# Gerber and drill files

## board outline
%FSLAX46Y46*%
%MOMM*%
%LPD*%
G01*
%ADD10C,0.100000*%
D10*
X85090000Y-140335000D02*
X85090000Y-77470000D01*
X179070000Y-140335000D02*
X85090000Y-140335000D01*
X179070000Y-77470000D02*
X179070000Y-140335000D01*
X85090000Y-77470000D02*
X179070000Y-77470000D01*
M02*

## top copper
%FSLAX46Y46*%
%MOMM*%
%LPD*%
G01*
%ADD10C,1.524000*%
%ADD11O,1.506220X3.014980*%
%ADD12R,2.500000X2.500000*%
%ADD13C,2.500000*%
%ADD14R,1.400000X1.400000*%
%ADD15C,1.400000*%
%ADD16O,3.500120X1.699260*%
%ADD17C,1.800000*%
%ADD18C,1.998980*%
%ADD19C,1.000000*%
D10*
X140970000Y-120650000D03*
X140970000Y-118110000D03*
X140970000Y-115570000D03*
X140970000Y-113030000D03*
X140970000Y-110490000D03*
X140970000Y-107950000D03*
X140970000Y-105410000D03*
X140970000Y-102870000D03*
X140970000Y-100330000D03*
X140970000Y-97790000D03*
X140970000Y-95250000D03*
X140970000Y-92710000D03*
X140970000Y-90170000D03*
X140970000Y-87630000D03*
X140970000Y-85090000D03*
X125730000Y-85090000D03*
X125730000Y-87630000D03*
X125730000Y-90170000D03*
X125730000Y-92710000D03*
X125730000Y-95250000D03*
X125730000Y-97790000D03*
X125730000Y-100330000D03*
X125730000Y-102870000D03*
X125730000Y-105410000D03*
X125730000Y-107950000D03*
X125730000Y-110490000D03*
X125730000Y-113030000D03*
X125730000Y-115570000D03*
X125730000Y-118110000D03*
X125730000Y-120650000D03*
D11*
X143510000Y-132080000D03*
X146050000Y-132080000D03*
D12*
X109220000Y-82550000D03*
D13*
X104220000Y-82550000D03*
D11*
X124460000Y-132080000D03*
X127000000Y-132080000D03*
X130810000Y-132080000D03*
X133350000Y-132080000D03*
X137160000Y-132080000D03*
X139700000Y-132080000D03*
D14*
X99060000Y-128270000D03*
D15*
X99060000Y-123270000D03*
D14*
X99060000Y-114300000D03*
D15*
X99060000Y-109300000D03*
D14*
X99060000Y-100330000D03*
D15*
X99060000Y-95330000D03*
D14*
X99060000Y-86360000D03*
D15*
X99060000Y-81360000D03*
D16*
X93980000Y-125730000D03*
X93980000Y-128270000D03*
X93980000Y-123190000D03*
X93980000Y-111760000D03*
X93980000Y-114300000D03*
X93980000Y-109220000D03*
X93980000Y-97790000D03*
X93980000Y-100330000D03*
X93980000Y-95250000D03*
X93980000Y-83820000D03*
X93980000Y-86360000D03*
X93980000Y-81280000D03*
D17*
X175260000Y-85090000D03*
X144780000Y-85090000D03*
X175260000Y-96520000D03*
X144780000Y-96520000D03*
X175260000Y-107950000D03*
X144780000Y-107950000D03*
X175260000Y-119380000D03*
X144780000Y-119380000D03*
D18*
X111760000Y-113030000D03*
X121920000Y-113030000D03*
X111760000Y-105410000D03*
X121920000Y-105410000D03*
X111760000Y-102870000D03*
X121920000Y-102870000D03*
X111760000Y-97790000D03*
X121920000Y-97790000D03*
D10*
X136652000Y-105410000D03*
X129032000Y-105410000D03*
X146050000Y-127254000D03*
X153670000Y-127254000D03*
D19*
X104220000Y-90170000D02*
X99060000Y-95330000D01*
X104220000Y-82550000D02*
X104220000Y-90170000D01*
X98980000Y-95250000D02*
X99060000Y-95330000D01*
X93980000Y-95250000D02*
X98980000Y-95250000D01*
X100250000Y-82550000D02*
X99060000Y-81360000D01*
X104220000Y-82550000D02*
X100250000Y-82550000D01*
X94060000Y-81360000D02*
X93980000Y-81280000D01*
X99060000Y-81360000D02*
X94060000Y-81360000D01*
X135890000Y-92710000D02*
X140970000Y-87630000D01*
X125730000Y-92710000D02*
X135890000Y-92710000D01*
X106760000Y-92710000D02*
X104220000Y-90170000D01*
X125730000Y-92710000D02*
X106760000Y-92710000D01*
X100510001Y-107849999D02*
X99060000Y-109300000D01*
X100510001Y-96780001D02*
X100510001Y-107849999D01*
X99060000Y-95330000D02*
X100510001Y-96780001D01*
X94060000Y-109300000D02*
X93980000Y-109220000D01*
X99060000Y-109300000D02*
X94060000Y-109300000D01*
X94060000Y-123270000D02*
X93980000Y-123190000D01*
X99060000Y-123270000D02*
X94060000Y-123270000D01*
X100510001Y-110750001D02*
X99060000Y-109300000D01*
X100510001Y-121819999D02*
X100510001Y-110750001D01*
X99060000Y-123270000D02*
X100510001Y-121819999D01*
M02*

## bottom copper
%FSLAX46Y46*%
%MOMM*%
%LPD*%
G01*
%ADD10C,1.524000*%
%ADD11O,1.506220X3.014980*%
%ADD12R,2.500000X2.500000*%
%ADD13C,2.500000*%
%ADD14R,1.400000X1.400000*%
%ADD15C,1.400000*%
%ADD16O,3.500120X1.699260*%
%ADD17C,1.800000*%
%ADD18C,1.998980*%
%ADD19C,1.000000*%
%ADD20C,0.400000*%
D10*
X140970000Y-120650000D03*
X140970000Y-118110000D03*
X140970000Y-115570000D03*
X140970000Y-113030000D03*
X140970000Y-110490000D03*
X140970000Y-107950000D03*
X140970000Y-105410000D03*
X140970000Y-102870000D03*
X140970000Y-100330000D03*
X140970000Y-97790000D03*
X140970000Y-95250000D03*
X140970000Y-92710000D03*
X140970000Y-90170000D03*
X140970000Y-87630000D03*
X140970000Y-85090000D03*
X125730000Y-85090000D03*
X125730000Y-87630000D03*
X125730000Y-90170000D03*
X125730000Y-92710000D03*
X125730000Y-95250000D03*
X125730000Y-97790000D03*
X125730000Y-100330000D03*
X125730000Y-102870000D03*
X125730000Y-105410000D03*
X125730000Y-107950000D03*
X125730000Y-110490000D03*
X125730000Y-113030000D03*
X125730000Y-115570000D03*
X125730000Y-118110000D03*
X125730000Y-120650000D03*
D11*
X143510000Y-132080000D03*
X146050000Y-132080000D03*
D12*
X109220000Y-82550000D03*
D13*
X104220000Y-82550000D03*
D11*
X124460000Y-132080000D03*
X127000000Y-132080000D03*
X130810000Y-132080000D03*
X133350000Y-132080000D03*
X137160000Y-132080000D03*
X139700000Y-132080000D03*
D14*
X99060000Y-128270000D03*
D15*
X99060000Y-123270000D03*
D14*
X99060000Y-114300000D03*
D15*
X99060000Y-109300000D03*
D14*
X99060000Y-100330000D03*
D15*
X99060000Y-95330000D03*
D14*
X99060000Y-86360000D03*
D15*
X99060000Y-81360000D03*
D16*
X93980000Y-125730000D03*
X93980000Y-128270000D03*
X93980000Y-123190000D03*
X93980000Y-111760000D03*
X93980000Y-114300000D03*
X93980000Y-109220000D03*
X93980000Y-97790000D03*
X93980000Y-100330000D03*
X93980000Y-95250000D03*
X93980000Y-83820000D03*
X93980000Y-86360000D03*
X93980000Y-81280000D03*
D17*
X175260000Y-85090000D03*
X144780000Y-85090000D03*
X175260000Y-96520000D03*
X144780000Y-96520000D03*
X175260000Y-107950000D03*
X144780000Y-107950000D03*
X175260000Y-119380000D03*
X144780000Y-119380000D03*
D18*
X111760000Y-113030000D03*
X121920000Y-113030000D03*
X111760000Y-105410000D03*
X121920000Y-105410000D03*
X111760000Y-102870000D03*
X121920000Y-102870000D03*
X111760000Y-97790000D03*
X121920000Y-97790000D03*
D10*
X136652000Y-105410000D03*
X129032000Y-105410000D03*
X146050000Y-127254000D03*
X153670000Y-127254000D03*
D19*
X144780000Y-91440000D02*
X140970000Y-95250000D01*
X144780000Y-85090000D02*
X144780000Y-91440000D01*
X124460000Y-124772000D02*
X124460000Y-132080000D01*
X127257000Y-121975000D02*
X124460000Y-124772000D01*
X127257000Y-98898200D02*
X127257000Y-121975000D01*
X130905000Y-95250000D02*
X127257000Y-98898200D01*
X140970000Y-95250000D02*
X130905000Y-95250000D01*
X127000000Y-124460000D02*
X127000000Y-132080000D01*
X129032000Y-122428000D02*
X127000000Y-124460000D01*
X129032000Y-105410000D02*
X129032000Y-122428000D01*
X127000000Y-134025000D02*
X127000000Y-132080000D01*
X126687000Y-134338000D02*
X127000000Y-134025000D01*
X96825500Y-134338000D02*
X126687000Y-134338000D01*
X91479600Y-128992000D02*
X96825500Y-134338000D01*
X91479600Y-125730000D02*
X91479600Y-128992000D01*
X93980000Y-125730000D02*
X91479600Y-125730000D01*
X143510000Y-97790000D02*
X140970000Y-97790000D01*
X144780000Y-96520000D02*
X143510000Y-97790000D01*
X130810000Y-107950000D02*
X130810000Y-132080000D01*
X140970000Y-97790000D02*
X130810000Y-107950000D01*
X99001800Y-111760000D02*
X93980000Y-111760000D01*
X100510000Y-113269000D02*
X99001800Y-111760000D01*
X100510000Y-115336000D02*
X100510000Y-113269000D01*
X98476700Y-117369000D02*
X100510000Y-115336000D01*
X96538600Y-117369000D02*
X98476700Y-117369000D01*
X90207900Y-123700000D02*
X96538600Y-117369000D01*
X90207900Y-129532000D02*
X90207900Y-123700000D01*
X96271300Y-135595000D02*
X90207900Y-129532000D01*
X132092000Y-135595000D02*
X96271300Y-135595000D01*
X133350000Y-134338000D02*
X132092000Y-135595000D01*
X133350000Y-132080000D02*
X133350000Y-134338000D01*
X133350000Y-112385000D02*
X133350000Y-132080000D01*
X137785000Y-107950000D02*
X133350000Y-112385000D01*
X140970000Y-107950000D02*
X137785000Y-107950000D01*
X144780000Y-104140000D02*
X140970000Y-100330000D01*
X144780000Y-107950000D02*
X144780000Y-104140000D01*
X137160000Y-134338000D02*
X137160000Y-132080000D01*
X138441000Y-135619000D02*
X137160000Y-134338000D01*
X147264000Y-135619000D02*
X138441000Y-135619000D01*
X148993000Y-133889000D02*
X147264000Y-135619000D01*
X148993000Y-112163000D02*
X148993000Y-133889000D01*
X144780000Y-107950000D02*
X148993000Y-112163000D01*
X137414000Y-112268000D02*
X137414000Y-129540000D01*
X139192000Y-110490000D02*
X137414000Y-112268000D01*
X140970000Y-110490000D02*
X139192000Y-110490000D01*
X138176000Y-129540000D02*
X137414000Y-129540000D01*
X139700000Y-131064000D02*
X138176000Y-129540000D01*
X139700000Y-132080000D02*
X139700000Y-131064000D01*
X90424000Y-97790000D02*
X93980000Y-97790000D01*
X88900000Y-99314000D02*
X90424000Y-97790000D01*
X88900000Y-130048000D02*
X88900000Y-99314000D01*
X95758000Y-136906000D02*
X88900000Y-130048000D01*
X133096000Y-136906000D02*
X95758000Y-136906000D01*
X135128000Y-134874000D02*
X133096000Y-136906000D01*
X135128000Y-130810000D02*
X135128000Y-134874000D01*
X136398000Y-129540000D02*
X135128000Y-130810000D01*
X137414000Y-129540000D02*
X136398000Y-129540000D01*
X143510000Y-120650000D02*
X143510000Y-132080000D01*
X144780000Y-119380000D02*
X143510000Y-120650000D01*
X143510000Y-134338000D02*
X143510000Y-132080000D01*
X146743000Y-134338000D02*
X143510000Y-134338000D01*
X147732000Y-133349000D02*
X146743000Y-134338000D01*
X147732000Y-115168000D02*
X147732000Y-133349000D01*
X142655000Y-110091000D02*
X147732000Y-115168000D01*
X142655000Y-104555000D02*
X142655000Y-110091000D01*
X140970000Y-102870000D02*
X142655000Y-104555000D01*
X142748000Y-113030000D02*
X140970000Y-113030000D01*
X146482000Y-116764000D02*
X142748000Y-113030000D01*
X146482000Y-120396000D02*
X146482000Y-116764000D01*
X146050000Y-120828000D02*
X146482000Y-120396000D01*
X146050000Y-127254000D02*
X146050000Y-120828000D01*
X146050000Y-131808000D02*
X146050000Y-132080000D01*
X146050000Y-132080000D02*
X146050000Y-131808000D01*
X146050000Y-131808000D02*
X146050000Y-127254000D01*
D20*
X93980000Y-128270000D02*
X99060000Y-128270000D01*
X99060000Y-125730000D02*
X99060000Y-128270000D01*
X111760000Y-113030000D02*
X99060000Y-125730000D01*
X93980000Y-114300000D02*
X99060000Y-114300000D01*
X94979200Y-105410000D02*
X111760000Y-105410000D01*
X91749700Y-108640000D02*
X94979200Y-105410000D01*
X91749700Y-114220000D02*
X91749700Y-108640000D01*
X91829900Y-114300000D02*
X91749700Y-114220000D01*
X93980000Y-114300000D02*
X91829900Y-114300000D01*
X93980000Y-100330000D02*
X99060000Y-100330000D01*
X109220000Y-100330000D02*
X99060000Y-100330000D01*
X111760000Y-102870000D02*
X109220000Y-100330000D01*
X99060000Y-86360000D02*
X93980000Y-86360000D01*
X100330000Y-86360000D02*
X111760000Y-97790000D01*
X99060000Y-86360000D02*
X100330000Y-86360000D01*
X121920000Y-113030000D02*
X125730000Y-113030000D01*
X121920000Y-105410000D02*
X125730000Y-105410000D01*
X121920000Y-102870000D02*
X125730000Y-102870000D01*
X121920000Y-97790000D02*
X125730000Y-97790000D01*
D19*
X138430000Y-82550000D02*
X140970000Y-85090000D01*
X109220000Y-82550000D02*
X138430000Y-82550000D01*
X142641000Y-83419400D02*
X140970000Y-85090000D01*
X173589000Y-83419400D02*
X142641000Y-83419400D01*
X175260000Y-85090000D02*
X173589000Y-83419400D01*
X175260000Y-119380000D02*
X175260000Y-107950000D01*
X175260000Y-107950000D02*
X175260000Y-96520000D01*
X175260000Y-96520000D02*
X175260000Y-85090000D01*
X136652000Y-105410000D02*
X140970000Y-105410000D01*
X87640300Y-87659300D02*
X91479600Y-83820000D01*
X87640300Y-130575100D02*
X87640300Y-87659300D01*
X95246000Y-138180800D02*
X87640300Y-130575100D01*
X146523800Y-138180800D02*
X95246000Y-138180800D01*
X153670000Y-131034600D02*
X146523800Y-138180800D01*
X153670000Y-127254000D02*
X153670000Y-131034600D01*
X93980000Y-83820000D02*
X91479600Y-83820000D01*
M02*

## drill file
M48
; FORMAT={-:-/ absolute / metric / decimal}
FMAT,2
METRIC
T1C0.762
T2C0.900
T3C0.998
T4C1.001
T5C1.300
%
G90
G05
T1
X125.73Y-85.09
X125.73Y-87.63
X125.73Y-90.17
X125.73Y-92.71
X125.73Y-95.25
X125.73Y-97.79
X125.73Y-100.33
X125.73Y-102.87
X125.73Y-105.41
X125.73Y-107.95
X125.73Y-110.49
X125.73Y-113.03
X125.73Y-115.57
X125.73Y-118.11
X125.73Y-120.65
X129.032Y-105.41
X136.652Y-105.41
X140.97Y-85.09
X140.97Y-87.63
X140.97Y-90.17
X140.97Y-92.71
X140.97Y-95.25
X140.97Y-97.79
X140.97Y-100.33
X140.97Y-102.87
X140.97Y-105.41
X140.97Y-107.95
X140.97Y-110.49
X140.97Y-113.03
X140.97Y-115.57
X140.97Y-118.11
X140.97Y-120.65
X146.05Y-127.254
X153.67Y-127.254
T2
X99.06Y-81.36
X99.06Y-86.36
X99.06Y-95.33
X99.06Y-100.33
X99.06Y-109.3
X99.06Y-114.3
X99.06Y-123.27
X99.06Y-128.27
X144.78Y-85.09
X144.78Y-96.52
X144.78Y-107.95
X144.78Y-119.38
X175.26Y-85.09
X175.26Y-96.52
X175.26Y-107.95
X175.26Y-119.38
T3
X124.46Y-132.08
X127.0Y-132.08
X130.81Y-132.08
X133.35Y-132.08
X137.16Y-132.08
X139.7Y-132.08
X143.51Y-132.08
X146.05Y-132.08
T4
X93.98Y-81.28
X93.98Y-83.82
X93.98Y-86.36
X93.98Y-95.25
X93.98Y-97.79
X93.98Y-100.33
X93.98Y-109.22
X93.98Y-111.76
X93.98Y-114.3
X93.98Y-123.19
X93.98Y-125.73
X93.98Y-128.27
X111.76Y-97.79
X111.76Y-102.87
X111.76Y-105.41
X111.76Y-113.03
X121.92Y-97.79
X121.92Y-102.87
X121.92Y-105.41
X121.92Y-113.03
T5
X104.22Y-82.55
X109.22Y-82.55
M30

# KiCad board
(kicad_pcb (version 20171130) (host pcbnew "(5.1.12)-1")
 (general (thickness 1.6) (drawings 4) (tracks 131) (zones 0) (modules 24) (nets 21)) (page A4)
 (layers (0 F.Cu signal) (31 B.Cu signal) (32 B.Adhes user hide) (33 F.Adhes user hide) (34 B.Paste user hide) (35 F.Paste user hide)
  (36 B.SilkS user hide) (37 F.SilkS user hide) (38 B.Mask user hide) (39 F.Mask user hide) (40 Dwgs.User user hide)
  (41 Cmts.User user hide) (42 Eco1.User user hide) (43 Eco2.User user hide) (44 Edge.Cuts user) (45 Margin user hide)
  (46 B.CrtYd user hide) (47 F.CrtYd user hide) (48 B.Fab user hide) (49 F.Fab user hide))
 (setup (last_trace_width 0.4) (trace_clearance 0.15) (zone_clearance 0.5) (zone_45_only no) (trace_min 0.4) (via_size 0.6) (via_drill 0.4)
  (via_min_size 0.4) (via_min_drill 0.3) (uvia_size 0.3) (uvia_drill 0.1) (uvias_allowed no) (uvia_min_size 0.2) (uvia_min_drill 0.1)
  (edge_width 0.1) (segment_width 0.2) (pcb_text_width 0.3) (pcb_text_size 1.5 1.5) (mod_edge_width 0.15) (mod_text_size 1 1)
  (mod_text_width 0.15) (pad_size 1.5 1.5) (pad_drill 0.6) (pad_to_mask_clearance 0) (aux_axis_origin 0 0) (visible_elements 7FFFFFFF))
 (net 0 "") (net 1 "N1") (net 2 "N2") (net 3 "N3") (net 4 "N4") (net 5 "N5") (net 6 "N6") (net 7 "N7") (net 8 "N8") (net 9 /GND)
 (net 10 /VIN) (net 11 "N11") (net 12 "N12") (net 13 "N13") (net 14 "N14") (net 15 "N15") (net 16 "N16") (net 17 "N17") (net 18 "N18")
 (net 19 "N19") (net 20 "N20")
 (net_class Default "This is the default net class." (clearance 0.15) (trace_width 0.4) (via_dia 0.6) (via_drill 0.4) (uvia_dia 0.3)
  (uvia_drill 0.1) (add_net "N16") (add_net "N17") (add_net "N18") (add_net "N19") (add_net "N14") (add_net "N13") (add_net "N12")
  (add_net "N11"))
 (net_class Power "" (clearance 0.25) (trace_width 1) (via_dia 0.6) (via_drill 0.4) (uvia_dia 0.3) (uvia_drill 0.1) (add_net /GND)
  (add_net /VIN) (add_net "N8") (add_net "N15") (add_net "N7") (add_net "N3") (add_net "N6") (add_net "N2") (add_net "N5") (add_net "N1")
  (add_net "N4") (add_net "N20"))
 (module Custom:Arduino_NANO (layer F.Cu) (at 140.97 120.65 90)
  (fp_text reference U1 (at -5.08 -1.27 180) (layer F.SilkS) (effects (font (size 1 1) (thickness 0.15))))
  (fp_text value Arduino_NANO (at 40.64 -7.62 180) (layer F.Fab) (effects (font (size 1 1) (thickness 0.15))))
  (pad 1 thru_hole circle (at 0 0 90) (size 1.524 1.524) (drill 0.762) (layers *.Cu *.Mask))
  (pad 2 thru_hole circle (at 2.54 0 90) (size 1.524 1.524) (drill 0.762) (layers *.Cu *.Mask))
  (pad 3 thru_hole circle (at 5.08 0 90) (size 1.524 1.524) (drill 0.762) (layers *.Cu *.Mask))
  (pad 4 thru_hole circle (at 7.62 0 90) (size 1.524 1.524) (drill 0.762) (layers *.Cu *.Mask) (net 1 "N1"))
  (pad 5 thru_hole circle (at 10.16 0 90) (size 1.524 1.524) (drill 0.762) (layers *.Cu *.Mask) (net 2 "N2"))
  (pad 6 thru_hole circle (at 12.7 0 90) (size 1.524 1.524) (drill 0.762) (layers *.Cu *.Mask) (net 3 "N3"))
  (pad 7 thru_hole circle (at 15.24 0 90) (size 1.524 1.524) (drill 0.762) (layers *.Cu *.Mask) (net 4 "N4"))
  (pad 8 thru_hole circle (at 17.78 0 90) (size 1.524 1.524) (drill 0.762) (layers *.Cu *.Mask) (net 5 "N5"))
  (pad 9 thru_hole circle (at 20.32 0 90) (size 1.524 1.524) (drill 0.762) (layers *.Cu *.Mask) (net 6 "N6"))
  (pad 10 thru_hole circle (at 22.86 0 90) (size 1.524 1.524) (drill 0.762) (layers *.Cu *.Mask) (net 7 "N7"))
  (pad 11 thru_hole circle (at 25.4 0 90) (size 1.524 1.524) (drill 0.762) (layers *.Cu *.Mask) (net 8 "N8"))
  (pad 12 thru_hole circle (at 27.94 0 90) (size 1.524 1.524) (drill 0.762) (layers *.Cu *.Mask))
  (pad 13 thru_hole circle (at 30.48 0 90) (size 1.524 1.524) (drill 0.762) (layers *.Cu *.Mask))
  (pad 14 thru_hole circle (at 33.02 0 90) (size 1.524 1.524) (drill 0.762) (layers *.Cu *.Mask) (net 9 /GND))
  (pad 15 thru_hole circle (at 35.56 0 90) (size 1.524 1.524) (drill 0.762) (layers *.Cu *.Mask) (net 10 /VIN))
  (pad 16 thru_hole circle (at 35.56 -15.24 90) (size 1.524 1.524) (drill 0.762) (layers *.Cu *.Mask))
  (pad 17 thru_hole circle (at 33.02 -15.24 90) (size 1.524 1.524) (drill 0.762) (layers *.Cu *.Mask))
  (pad 18 thru_hole circle (at 30.48 -15.24 90) (size 1.524 1.524) (drill 0.762) (layers *.Cu *.Mask))
  (pad 19 thru_hole circle (at 27.94 -15.24 90) (size 1.524 1.524) (drill 0.762) (layers *.Cu *.Mask) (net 9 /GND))
  (pad 20 thru_hole circle (at 25.4 -15.24 90) (size 1.524 1.524) (drill 0.762) (layers *.Cu *.Mask))
  (pad 21 thru_hole circle (at 22.86 -15.24 90) (size 1.524 1.524) (drill 0.762) (layers *.Cu *.Mask) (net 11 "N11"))
  (pad 22 thru_hole circle (at 20.32 -15.24 90) (size 1.524 1.524) (drill 0.762) (layers *.Cu *.Mask))
  (pad 23 thru_hole circle (at 17.78 -15.24 90) (size 1.524 1.524) (drill 0.762) (layers *.Cu *.Mask) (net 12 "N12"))
  (pad 24 thru_hole circle (at 15.24 -15.24 90) (size 1.524 1.524) (drill 0.762) (layers *.Cu *.Mask) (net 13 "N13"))
  (pad 25 thru_hole circle (at 12.7 -15.24 90) (size 1.524 1.524) (drill 0.762) (layers *.Cu *.Mask))
  (pad 26 thru_hole circle (at 10.16 -15.24 90) (size 1.524 1.524) (drill 0.762) (layers *.Cu *.Mask))
  (pad 27 thru_hole circle (at 7.62 -15.24 90) (size 1.524 1.524) (drill 0.762) (layers *.Cu *.Mask) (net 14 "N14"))
  (pad 28 thru_hole circle (at 5.08 -15.24 90) (size 1.524 1.524) (drill 0.762) (layers *.Cu *.Mask))
  (pad 29 thru_hole circle (at 2.54 -15.24 90) (size 1.524 1.524) (drill 0.762) (layers *.Cu *.Mask))
  (pad 30 thru_hole circle (at 0 -15.24 90) (size 1.524 1.524) (drill 0.762) (layers *.Cu *.Mask)))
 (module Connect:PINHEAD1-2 (layer F.Cu) (at 144.78 132.08)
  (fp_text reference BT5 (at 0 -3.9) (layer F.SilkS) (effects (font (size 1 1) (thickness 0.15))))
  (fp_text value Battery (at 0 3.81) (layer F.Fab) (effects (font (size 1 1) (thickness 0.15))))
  (pad 1 thru_hole oval (at -1.27 0) (size 1.50622 3.01498) (drill 0.99822) (layers *.Cu *.Mask) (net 5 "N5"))
  (pad 2 thru_hole oval (at 1.27 0) (size 1.50622 3.01498) (drill 0.99822) (layers *.Cu *.Mask) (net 1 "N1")))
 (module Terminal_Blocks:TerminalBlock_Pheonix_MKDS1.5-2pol (layer F.Cu) (at 109.22 82.55 180)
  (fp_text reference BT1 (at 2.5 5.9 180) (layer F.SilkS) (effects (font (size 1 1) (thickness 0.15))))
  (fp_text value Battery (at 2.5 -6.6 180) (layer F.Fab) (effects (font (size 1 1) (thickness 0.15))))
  (pad 1 thru_hole rect (at 0 0 180) (size 2.5 2.5) (drill 1.3) (layers *.Cu *.Mask F.SilkS) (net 10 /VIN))
  (pad 2 thru_hole circle (at 5 0 180) (size 2.5 2.5) (drill 1.3) (layers *.Cu *.Mask F.SilkS) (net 9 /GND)))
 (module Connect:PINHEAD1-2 (layer F.Cu) (at 125.73 132.08)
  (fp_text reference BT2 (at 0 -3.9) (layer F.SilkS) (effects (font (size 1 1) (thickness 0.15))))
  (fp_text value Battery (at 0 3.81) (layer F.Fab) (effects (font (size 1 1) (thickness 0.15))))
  (pad 1 thru_hole oval (at -1.27 0) (size 1.50622 3.01498) (drill 0.99822) (layers *.Cu *.Mask) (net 8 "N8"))
  (pad 2 thru_hole oval (at 1.27 0) (size 1.50622 3.01498) (drill 0.99822) (layers *.Cu *.Mask) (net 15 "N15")))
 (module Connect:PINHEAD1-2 (layer F.Cu) (at 132.08 132.08)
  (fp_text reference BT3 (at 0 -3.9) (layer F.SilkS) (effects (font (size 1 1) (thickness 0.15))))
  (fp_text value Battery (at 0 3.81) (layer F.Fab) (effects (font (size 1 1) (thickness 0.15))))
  (pad 1 thru_hole oval (at -1.27 0) (size 1.50622 3.01498) (drill 0.99822) (layers *.Cu *.Mask) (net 7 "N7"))
  (pad 2 thru_hole oval (at 1.27 0) (size 1.50622 3.01498) (drill 0.99822) (layers *.Cu *.Mask) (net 3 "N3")))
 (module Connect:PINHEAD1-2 (layer F.Cu) (at 138.43 132.08)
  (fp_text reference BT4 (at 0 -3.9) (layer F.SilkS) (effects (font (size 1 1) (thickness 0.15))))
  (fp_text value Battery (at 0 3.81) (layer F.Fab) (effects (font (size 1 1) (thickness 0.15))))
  (pad 1 thru_hole oval (at -1.27 0) (size 1.50622 3.01498) (drill 0.99822) (layers *.Cu *.Mask) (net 6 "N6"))
  (pad 2 thru_hole oval (at 1.27 0) (size 1.50622 3.01498) (drill 0.99822) (layers *.Cu *.Mask) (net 2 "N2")))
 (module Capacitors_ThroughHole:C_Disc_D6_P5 (layer F.Cu) (at 99.06 128.27 90)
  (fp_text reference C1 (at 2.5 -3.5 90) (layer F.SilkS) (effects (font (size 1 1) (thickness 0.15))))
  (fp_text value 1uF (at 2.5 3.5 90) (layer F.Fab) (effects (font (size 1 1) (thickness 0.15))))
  (pad 1 thru_hole rect (at 0 0 90) (size 1.4 1.4) (drill 0.9) (layers *.Cu *.Mask F.SilkS) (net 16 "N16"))
  (pad 2 thru_hole circle (at 5 0 90) (size 1.4 1.4) (drill 0.9) (layers *.Cu *.Mask F.SilkS) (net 9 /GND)))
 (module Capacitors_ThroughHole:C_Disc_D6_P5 (layer F.Cu) (at 99.06 114.3 90)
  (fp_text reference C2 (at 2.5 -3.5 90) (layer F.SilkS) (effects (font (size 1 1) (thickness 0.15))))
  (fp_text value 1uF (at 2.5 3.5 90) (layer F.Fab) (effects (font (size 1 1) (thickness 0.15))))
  (pad 1 thru_hole rect (at 0 0 90) (size 1.4 1.4) (drill 0.9) (layers *.Cu *.Mask F.SilkS) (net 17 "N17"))
  (pad 2 thru_hole circle (at 5 0 90) (size 1.4 1.4) (drill 0.9) (layers *.Cu *.Mask F.SilkS) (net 9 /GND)))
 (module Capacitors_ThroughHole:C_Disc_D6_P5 (layer F.Cu) (at 99.06 100.33 90)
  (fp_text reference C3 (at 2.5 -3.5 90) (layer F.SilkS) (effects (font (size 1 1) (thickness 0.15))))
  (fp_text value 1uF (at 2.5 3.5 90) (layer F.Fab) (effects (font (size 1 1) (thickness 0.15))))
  (pad 1 thru_hole rect (at 0 0 90) (size 1.4 1.4) (drill 0.9) (layers *.Cu *.Mask F.SilkS) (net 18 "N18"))
  (pad 2 thru_hole circle (at 5 0 90) (size 1.4 1.4) (drill 0.9) (layers *.Cu *.Mask F.SilkS) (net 9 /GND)))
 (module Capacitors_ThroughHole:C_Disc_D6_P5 (layer F.Cu) (at 99.06 86.36 90)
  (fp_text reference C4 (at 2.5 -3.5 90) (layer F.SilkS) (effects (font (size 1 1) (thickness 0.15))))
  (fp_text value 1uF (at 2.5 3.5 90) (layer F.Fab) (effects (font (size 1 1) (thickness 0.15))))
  (pad 1 thru_hole rect (at 0 0 90) (size 1.4 1.4) (drill 0.9) (layers *.Cu *.Mask F.SilkS) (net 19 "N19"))
  (pad 2 thru_hole circle (at 5 0 90) (size 1.4 1.4) (drill 0.9) (layers *.Cu *.Mask F.SilkS) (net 9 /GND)))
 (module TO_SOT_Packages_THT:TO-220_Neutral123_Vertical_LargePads (layer F.Cu) (at 93.98 125.73 90)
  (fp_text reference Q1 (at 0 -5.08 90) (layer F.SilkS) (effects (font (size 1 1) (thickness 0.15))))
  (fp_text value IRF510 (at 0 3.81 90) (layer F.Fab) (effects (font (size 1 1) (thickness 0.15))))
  (pad 2 thru_hole oval (at 0 0 180) (size 3.50012 1.69926) (drill 1.00076) (layers *.Cu *.Mask F.SilkS) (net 15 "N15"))
  (pad 1 thru_hole oval (at -2.54 0 180) (size 3.50012 1.69926) (drill 1.00076) (layers *.Cu *.Mask F.SilkS) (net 16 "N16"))
  (pad 3 thru_hole oval (at 2.54 0 180) (size 3.50012 1.69926) (drill 1.00076) (layers *.Cu *.Mask F.SilkS) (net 9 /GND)))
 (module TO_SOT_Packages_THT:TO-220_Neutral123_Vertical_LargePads (layer F.Cu) (at 93.98 111.76 90)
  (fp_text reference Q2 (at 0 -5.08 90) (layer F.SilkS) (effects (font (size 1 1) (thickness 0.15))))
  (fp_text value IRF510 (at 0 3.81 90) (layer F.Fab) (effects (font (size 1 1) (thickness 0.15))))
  (pad 2 thru_hole oval (at 0 0 180) (size 3.50012 1.69926) (drill 1.00076) (layers *.Cu *.Mask F.SilkS) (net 3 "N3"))
  (pad 1 thru_hole oval (at -2.54 0 180) (size 3.50012 1.69926) (drill 1.00076) (layers *.Cu *.Mask F.SilkS) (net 17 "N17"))
  (pad 3 thru_hole oval (at 2.54 0 180) (size 3.50012 1.69926) (drill 1.00076) (layers *.Cu *.Mask F.SilkS) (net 9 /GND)))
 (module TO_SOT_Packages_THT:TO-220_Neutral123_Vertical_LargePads (layer F.Cu) (at 93.98 97.79 90)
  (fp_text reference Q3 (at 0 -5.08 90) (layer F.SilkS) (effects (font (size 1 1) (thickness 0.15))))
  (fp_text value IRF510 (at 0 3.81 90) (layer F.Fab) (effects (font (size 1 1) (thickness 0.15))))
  (pad 2 thru_hole oval (at 0 0 180) (size 3.50012 1.69926) (drill 1.00076) (layers *.Cu *.Mask F.SilkS) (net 2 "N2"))
  (pad 1 thru_hole oval (at -2.54 0 180) (size 3.50012 1.69926) (drill 1.00076) (layers *.Cu *.Mask F.SilkS) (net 18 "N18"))
  (pad 3 thru_hole oval (at 2.54 0 180) (size 3.50012 1.69926) (drill 1.00076) (layers *.Cu *.Mask F.SilkS) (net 9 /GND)))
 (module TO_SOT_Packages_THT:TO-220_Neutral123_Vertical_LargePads (layer F.Cu) (at 93.98 83.82 90)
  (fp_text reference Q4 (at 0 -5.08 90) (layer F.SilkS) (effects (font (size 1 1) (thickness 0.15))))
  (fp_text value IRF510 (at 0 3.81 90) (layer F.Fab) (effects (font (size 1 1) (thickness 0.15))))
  (pad 2 thru_hole oval (at 0 0 180) (size 3.50012 1.69926) (drill 1.00076) (layers *.Cu *.Mask F.SilkS) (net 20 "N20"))
  (pad 1 thru_hole oval (at -2.54 0 180) (size 3.50012 1.69926) (drill 1.00076) (layers *.Cu *.Mask F.SilkS) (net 19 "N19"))
  (pad 3 thru_hole oval (at 2.54 0 180) (size 3.50012 1.69926) (drill 1.00076) (layers *.Cu *.Mask F.SilkS) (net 9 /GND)))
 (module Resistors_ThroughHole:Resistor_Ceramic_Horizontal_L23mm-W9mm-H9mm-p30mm (layer F.Cu) (at 160.02 85.09 180)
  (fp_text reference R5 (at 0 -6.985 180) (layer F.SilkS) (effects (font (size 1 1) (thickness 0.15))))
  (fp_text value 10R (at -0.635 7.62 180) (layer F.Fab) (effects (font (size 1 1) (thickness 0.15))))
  (pad 1 thru_hole circle (at -15.24 0) (size 1.8 1.8) (drill 0.9) (layers *.Cu *.Mask F.SilkS) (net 10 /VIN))
  (pad 2 thru_hole circle (at 15.24 0) (size 1.8 1.8) (drill 0.9) (layers *.Cu *.Mask F.SilkS) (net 8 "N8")))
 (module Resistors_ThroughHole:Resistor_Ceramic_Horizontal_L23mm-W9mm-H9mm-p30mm (layer F.Cu) (at 160.02 96.52 180)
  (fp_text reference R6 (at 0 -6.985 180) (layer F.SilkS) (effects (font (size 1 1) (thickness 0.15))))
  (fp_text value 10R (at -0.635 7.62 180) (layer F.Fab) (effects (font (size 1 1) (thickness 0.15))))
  (pad 1 thru_hole circle (at -15.24 0) (size 1.8 1.8) (drill 0.9) (layers *.Cu *.Mask F.SilkS) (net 10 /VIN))
  (pad 2 thru_hole circle (at 15.24 0) (size 1.8 1.8) (drill 0.9) (layers *.Cu *.Mask F.SilkS) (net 7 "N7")))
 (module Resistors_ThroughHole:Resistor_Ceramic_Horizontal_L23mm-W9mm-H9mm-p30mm (layer F.Cu) (at 160.02 107.95 180)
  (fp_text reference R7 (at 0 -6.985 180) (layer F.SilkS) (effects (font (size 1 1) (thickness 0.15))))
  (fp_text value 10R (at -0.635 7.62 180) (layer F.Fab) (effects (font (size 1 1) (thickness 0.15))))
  (pad 1 thru_hole circle (at -15.24 0) (size 1.8 1.8) (drill 0.9) (layers *.Cu *.Mask F.SilkS) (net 10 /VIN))
  (pad 2 thru_hole circle (at 15.24 0) (size 1.8 1.8) (drill 0.9) (layers *.Cu *.Mask F.SilkS) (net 6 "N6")))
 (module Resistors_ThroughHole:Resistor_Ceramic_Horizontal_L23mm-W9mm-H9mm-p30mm (layer F.Cu) (at 160.02 119.38 180)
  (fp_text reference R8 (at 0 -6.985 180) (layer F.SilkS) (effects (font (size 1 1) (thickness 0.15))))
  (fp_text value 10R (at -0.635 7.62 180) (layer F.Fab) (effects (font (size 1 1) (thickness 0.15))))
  (pad 1 thru_hole circle (at -15.24 0) (size 1.8 1.8) (drill 0.9) (layers *.Cu *.Mask F.SilkS) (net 10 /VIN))
  (pad 2 thru_hole circle (at 15.24 0) (size 1.8 1.8) (drill 0.9) (layers *.Cu *.Mask F.SilkS) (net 5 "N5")))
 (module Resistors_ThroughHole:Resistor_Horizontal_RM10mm (layer F.Cu) (at 111.76 113.03)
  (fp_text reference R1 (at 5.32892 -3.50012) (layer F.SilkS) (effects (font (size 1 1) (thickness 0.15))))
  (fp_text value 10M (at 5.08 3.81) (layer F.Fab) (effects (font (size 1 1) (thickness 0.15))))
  (pad 1 thru_hole circle (at 0 0) (size 1.99898 1.99898) (drill 1.00076) (layers *.Cu *.SilkS *.Mask) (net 16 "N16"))
  (pad 2 thru_hole circle (at 10.16 0) (size 1.99898 1.99898) (drill 1.00076) (layers *.Cu *.SilkS *.Mask) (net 14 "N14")))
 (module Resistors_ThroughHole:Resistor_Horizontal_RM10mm (layer F.Cu) (at 111.76 105.41)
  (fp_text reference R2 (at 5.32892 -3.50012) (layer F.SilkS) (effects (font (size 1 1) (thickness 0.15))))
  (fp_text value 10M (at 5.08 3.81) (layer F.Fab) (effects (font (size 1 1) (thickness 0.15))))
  (pad 1 thru_hole circle (at 0 0) (size 1.99898 1.99898) (drill 1.00076) (layers *.Cu *.SilkS *.Mask) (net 17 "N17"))
  (pad 2 thru_hole circle (at 10.16 0) (size 1.99898 1.99898) (drill 1.00076) (layers *.Cu *.SilkS *.Mask) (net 13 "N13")))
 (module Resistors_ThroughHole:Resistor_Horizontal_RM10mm (layer F.Cu) (at 111.76 102.87)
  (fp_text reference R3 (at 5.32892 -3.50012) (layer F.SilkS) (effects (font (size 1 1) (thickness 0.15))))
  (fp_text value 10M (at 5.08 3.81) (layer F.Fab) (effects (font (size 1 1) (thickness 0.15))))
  (pad 1 thru_hole circle (at 0 0) (size 1.99898 1.99898) (drill 1.00076) (layers *.Cu *.SilkS *.Mask) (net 18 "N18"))
  (pad 2 thru_hole circle (at 10.16 0) (size 1.99898 1.99898) (drill 1.00076) (layers *.Cu *.SilkS *.Mask) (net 12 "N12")))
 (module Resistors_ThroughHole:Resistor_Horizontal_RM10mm (layer F.Cu) (at 111.76 97.79)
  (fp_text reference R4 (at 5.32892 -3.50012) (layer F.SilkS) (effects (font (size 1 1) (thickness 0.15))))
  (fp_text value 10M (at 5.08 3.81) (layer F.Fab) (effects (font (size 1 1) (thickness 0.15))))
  (pad 1 thru_hole circle (at 0 0) (size 1.99898 1.99898) (drill 1.00076) (layers *.Cu *.SilkS *.Mask) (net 19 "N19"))
  (pad 2 thru_hole circle (at 10.16 0) (size 1.99898 1.99898) (drill 1.00076) (layers *.Cu *.SilkS *.Mask) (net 11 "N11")))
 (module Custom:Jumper (layer F.Cu) (at 132.842 105.41 180)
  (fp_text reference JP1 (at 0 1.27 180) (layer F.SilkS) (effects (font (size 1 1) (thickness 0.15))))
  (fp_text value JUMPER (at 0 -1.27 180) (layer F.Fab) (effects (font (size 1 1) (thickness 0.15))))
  (pad 1 thru_hole circle (at -3.81 0 180) (size 1.524 1.524) (drill 0.762) (layers *.Cu *.Mask) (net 4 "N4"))
  (pad 2 thru_hole circle (at 3.81 0 180) (size 1.524 1.524) (drill 0.762) (layers *.Cu *.Mask) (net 15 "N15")))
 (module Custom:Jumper (layer F.Cu) (at 149.86 127.254)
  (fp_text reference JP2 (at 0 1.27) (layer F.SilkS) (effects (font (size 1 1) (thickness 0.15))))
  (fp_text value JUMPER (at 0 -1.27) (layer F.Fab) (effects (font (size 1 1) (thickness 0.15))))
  (pad 1 thru_hole circle (at -3.81 0) (size 1.524 1.524) (drill 0.762) (layers *.Cu *.Mask) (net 1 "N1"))
  (pad 2 thru_hole circle (at 3.81 0) (size 1.524 1.524) (drill 0.762) (layers *.Cu *.Mask) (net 20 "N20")))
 (gr_line (start 85.09 140.335) (end 85.09 77.47) (angle 90) (layer Edge.Cuts) (width 0.1))
 (gr_line (start 179.07 140.335) (end 85.09 140.335) (angle 90) (layer Edge.Cuts) (width 0.1))
 (gr_line (start 179.07 77.47) (end 179.07 140.335) (angle 90) (layer Edge.Cuts) (width 0.1))
 (gr_line (start 85.09 77.47) (end 179.07 77.47) (angle 90) (layer Edge.Cuts) (width 0.1))
 (segment (start 104.22 90.17) (end 99.06 95.33) (width 1) (layer F.Cu) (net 9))
 (segment (start 104.22 82.55) (end 104.22 90.17) (width 1) (layer F.Cu) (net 9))
 (segment (start 98.98 95.25) (end 99.06 95.33) (width 1) (layer F.Cu) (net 9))
 (segment (start 93.98 95.25) (end 98.98 95.25) (width 1) (layer F.Cu) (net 9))
 (segment (start 100.25 82.55) (end 99.06 81.36) (width 1) (layer F.Cu) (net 9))
 (segment (start 104.22 82.55) (end 100.25 82.55) (width 1) (layer F.Cu) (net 9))
 (segment (start 94.06 81.36) (end 93.98 81.28) (width 1) (layer F.Cu) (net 9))
 (segment (start 99.06 81.36) (end 94.06 81.36) (width 1) (layer F.Cu) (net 9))
 (segment (start 135.89 92.71) (end 140.97 87.63) (width 1) (layer F.Cu) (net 9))
 (segment (start 125.73 92.71) (end 135.89 92.71) (width 1) (layer F.Cu) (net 9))
 (segment (start 106.76 92.71) (end 104.22 90.17) (width 1) (layer F.Cu) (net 9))
 (segment (start 125.73 92.71) (end 106.76 92.71) (width 1) (layer F.Cu) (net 9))
 (segment (start 100.510001 107.849999) (end 99.06 109.3) (width 1) (layer F.Cu) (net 9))
 (segment (start 100.510001 96.780001) (end 100.510001 107.849999) (width 1) (layer F.Cu) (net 9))
 (segment (start 99.06 95.33) (end 100.510001 96.780001) (width 1) (layer F.Cu) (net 9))
 (segment (start 94.06 109.3) (end 93.98 109.22) (width 1) (layer F.Cu) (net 9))
 (segment (start 99.06 109.3) (end 94.06 109.3) (width 1) (layer F.Cu) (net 9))
 (segment (start 94.06 123.27) (end 93.98 123.19) (width 1) (layer F.Cu) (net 9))
 (segment (start 99.06 123.27) (end 94.06 123.27) (width 1) (layer F.Cu) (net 9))
 (segment (start 100.510001 110.750001) (end 99.06 109.3) (width 1) (layer F.Cu) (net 9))
 (segment (start 100.510001 121.819999) (end 100.510001 110.750001) (width 1) (layer F.Cu) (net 9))
 (segment (start 99.06 123.27) (end 100.510001 121.819999) (width 1) (layer F.Cu) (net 9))
 (segment (start 144.78 91.44) (end 140.97 95.25) (width 1) (layer B.Cu) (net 8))
 (segment (start 144.78 85.09) (end 144.78 91.44) (width 1) (layer B.Cu) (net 8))
 (segment (start 124.46 124.772) (end 124.46 132.08) (width 1) (layer B.Cu) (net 8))
 (segment (start 127.257 121.975) (end 124.46 124.772) (width 1) (layer B.Cu) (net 8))
 (segment (start 127.257 98.8982) (end 127.257 121.975) (width 1) (layer B.Cu) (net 8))
 (segment (start 130.905 95.25) (end 127.257 98.8982) (width 1) (layer B.Cu) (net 8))
 (segment (start 140.97 95.25) (end 130.905 95.25) (width 1) (layer B.Cu) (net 8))
 (segment (start 127 124.46) (end 127 132.08) (width 1) (layer B.Cu) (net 15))
 (segment (start 129.032 122.428) (end 127 124.46) (width 1) (layer B.Cu) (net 15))
 (segment (start 129.032 105.41) (end 129.032 122.428) (width 1) (layer B.Cu) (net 15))
 (segment (start 127 134.025) (end 127 132.08) (width 1) (layer B.Cu) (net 15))
 (segment (start 126.687 134.338) (end 127 134.025) (width 1) (layer B.Cu) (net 15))
 (segment (start 96.8255 134.338) (end 126.687 134.338) (width 1) (layer B.Cu) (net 15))
 (segment (start 91.4796 128.992) (end 96.8255 134.338) (width 1) (layer B.Cu) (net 15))
 (segment (start 91.4796 125.73) (end 91.4796 128.992) (width 1) (layer B.Cu) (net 15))
 (segment (start 93.98 125.73) (end 91.4796 125.73) (width 1) (layer B.Cu) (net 15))
 (segment (start 143.51 97.79) (end 140.97 97.79) (width 1) (layer B.Cu) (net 7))
 (segment (start 144.78 96.52) (end 143.51 97.79) (width 1) (layer B.Cu) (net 7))
 (segment (start 130.81 107.95) (end 130.81 132.08) (width 1) (layer B.Cu) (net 7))
 (segment (start 140.97 97.79) (end 130.81 107.95) (width 1) (layer B.Cu) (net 7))
 (segment (start 99.0018 111.76) (end 93.98 111.76) (width 1) (layer B.Cu) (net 3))
 (segment (start 100.51 113.269) (end 99.0018 111.76) (width 1) (layer B.Cu) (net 3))
 (segment (start 100.51 115.336) (end 100.51 113.269) (width 1) (layer B.Cu) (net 3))
 (segment (start 98.4767 117.369) (end 100.51 115.336) (width 1) (layer B.Cu) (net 3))
 (segment (start 96.5386 117.369) (end 98.4767 117.369) (width 1) (layer B.Cu) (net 3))
 (segment (start 90.2079 123.7) (end 96.5386 117.369) (width 1) (layer B.Cu) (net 3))
 (segment (start 90.2079 129.532) (end 90.2079 123.7) (width 1) (layer B.Cu) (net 3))
 (segment (start 96.2713 135.595) (end 90.2079 129.532) (width 1) (layer B.Cu) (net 3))
 (segment (start 132.092 135.595) (end 96.2713 135.595) (width 1) (layer B.Cu) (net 3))
 (segment (start 133.35 134.338) (end 132.092 135.595) (width 1) (layer B.Cu) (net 3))
 (segment (start 133.35 132.08) (end 133.35 134.338) (width 1) (layer B.Cu) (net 3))
 (segment (start 133.35 112.385) (end 133.35 132.08) (width 1) (layer B.Cu) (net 3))
 (segment (start 137.785 107.95) (end 133.35 112.385) (width 1) (layer B.Cu) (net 3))
 (segment (start 140.97 107.95) (end 137.785 107.95) (width 1) (layer B.Cu) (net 3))
 (segment (start 144.78 104.14) (end 140.97 100.33) (width 1) (layer B.Cu) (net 6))
 (segment (start 144.78 107.95) (end 144.78 104.14) (width 1) (layer B.Cu) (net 6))
 (segment (start 137.16 134.338) (end 137.16 132.08) (width 1) (layer B.Cu) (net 6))
 (segment (start 138.441 135.619) (end 137.16 134.338) (width 1) (layer B.Cu) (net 6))
 (segment (start 147.264 135.619) (end 138.441 135.619) (width 1) (layer B.Cu) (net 6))
 (segment (start 148.993 133.889) (end 147.264 135.619) (width 1) (layer B.Cu) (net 6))
 (segment (start 148.993 112.163) (end 148.993 133.889) (width 1) (layer B.Cu) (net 6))
 (segment (start 144.78 107.95) (end 148.993 112.163) (width 1) (layer B.Cu) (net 6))
 (segment (start 137.414 112.268) (end 137.414 129.54) (width 1) (layer B.Cu) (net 2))
 (segment (start 139.192 110.49) (end 137.414 112.268) (width 1) (layer B.Cu) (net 2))
 (segment (start 140.97 110.49) (end 139.192 110.49) (width 1) (layer B.Cu) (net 2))
 (segment (start 138.176 129.54) (end 137.414 129.54) (width 1) (layer B.Cu) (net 2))
 (segment (start 139.7 131.064) (end 138.176 129.54) (width 1) (layer B.Cu) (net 2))
 (segment (start 139.7 132.08) (end 139.7 131.064) (width 1) (layer B.Cu) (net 2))
 (segment (start 90.424 97.79) (end 93.98 97.79) (width 1) (layer B.Cu) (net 2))
 (segment (start 88.9 99.314) (end 90.424 97.79) (width 1) (layer B.Cu) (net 2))
 (segment (start 88.9 130.048) (end 88.9 99.314) (width 1) (layer B.Cu) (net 2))
 (segment (start 95.758 136.906) (end 88.9 130.048) (width 1) (layer B.Cu) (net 2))
 (segment (start 133.096 136.906) (end 95.758 136.906) (width 1) (layer B.Cu) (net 2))
 (segment (start 135.128 134.874) (end 133.096 136.906) (width 1) (layer B.Cu) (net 2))
 (segment (start 135.128 130.81) (end 135.128 134.874) (width 1) (layer B.Cu) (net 2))
 (segment (start 136.398 129.54) (end 135.128 130.81) (width 1) (layer B.Cu) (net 2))
 (segment (start 137.414 129.54) (end 136.398 129.54) (width 1) (layer B.Cu) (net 2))
 (segment (start 143.51 120.65) (end 143.51 132.08) (width 1) (layer B.Cu) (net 5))
 (segment (start 144.78 119.38) (end 143.51 120.65) (width 1) (layer B.Cu) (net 5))
 (segment (start 143.51 134.338) (end 143.51 132.08) (width 1) (layer B.Cu) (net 5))
 (segment (start 146.743 134.338) (end 143.51 134.338) (width 1) (layer B.Cu) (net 5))
 (segment (start 147.732 133.349) (end 146.743 134.338) (width 1) (layer B.Cu) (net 5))
 (segment (start 147.732 115.168) (end 147.732 133.349) (width 1) (layer B.Cu) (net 5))
 (segment (start 142.655 110.091) (end 147.732 115.168) (width 1) (layer B.Cu) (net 5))
 (segment (start 142.655 104.555) (end 142.655 110.091) (width 1) (layer B.Cu) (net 5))
 (segment (start 140.97 102.87) (end 142.655 104.555) (width 1) (layer B.Cu) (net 5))
 (segment (start 142.748 113.03) (end 140.97 113.03) (width 1) (layer B.Cu) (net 1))
 (segment (start 146.482 116.764) (end 142.748 113.03) (width 1) (layer B.Cu) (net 1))
 (segment (start 146.482 120.396) (end 146.482 116.764) (width 1) (layer B.Cu) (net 1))
 (segment (start 146.05 120.828) (end 146.482 120.396) (width 1) (layer B.Cu) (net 1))
 (segment (start 146.05 127.254) (end 146.05 120.828) (width 1) (layer B.Cu) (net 1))
 (segment (start 146.05 131.808) (end 146.05 132.08) (width 1) (layer B.Cu) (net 1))
 (segment (start 146.05 132.08) (end 146.05 131.808) (width 1) (layer B.Cu) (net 1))
 (segment (start 146.05 131.808) (end 146.05 127.254) (width 1) (layer B.Cu) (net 1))
 (segment (start 93.98 128.27) (end 99.06 128.27) (width 0.4) (layer B.Cu) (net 16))
 (segment (start 99.06 125.73) (end 99.06 128.27) (width 0.4) (layer B.Cu) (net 16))
 (segment (start 111.76 113.03) (end 99.06 125.73) (width 0.4) (layer B.Cu) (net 16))
 (segment (start 93.98 114.3) (end 99.06 114.3) (width 0.4) (layer B.Cu) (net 17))
 (segment (start 94.9792 105.41) (end 111.76 105.41) (width 0.4) (layer B.Cu) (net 17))
 (segment (start 91.7497 108.64) (end 94.9792 105.41) (width 0.4) (layer B.Cu) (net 17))
 (segment (start 91.7497 114.22) (end 91.7497 108.64) (width 0.4) (layer B.Cu) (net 17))
 (segment (start 91.8299 114.3) (end 91.7497 114.22) (width 0.4) (layer B.Cu) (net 17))
 (segment (start 93.98 114.3) (end 91.8299 114.3) (width 0.4) (layer B.Cu) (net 17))
 (segment (start 93.98 100.33) (end 99.06 100.33) (width 0.4) (layer B.Cu) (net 18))
 (segment (start 109.22 100.33) (end 99.06 100.33) (width 0.4) (layer B.Cu) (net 18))
 (segment (start 111.76 102.87) (end 109.22 100.33) (width 0.4) (layer B.Cu) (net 18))
 (segment (start 99.06 86.36) (end 93.98 86.36) (width 0.4) (layer B.Cu) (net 19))
 (segment (start 100.33 86.36) (end 111.76 97.79) (width 0.4) (layer B.Cu) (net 19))
 (segment (start 99.06 86.36) (end 100.33 86.36) (width 0.4) (layer B.Cu) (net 19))
 (segment (start 121.92 113.03) (end 125.73 113.03) (width 0.4) (layer B.Cu) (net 14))
 (segment (start 121.92 105.41) (end 125.73 105.41) (width 0.4) (layer B.Cu) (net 13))
 (segment (start 121.92 102.87) (end 125.73 102.87) (width 0.4) (layer B.Cu) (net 12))
 (segment (start 121.92 97.79) (end 125.73 97.79) (width 0.4) (layer B.Cu) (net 11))
 (segment (start 138.43 82.55) (end 140.97 85.09) (width 1) (layer B.Cu) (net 10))
 (segment (start 109.22 82.55) (end 138.43 82.55) (width 1) (layer B.Cu) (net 10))
 (segment (start 142.641 83.4194) (end 140.97 85.09) (width 1) (layer B.Cu) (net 10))
 (segment (start 173.589 83.4194) (end 142.641 83.4194) (width 1) (layer B.Cu) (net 10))
 (segment (start 175.26 85.09) (end 173.589 83.4194) (width 1) (layer B.Cu) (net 10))
 (segment (start 175.26 119.38) (end 175.26 107.95) (width 1) (layer B.Cu) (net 10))
 (segment (start 175.26 107.95) (end 175.26 96.52) (width 1) (layer B.Cu) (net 10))
 (segment (start 175.26 96.52) (end 175.26 85.09) (width 1) (layer B.Cu) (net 10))
 (segment (start 136.652 105.41) (end 140.97 105.41) (width 1) (layer B.Cu) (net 4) (status C00000))
 (segment (start 87.6403 87.6593) (end 91.4796 83.82) (width 1) (layer B.Cu) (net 20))
 (segment (start 87.6403 130.5751) (end 87.6403 87.6593) (width 1) (layer B.Cu) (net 20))
 (segment (start 95.246 138.1808) (end 87.6403 130.5751) (width 1) (layer B.Cu) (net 20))
 (segment (start 146.5238 138.1808) (end 95.246 138.1808) (width 1) (layer B.Cu) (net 20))
 (segment (start 153.67 131.0346) (end 146.5238 138.1808) (width 1) (layer B.Cu) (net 20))
 (segment (start 153.67 127.254) (end 153.67 131.0346) (width 1) (layer B.Cu) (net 20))
 (segment (start 93.98 83.82) (end 91.4796 83.82) (width 1) (layer B.Cu) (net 20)))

